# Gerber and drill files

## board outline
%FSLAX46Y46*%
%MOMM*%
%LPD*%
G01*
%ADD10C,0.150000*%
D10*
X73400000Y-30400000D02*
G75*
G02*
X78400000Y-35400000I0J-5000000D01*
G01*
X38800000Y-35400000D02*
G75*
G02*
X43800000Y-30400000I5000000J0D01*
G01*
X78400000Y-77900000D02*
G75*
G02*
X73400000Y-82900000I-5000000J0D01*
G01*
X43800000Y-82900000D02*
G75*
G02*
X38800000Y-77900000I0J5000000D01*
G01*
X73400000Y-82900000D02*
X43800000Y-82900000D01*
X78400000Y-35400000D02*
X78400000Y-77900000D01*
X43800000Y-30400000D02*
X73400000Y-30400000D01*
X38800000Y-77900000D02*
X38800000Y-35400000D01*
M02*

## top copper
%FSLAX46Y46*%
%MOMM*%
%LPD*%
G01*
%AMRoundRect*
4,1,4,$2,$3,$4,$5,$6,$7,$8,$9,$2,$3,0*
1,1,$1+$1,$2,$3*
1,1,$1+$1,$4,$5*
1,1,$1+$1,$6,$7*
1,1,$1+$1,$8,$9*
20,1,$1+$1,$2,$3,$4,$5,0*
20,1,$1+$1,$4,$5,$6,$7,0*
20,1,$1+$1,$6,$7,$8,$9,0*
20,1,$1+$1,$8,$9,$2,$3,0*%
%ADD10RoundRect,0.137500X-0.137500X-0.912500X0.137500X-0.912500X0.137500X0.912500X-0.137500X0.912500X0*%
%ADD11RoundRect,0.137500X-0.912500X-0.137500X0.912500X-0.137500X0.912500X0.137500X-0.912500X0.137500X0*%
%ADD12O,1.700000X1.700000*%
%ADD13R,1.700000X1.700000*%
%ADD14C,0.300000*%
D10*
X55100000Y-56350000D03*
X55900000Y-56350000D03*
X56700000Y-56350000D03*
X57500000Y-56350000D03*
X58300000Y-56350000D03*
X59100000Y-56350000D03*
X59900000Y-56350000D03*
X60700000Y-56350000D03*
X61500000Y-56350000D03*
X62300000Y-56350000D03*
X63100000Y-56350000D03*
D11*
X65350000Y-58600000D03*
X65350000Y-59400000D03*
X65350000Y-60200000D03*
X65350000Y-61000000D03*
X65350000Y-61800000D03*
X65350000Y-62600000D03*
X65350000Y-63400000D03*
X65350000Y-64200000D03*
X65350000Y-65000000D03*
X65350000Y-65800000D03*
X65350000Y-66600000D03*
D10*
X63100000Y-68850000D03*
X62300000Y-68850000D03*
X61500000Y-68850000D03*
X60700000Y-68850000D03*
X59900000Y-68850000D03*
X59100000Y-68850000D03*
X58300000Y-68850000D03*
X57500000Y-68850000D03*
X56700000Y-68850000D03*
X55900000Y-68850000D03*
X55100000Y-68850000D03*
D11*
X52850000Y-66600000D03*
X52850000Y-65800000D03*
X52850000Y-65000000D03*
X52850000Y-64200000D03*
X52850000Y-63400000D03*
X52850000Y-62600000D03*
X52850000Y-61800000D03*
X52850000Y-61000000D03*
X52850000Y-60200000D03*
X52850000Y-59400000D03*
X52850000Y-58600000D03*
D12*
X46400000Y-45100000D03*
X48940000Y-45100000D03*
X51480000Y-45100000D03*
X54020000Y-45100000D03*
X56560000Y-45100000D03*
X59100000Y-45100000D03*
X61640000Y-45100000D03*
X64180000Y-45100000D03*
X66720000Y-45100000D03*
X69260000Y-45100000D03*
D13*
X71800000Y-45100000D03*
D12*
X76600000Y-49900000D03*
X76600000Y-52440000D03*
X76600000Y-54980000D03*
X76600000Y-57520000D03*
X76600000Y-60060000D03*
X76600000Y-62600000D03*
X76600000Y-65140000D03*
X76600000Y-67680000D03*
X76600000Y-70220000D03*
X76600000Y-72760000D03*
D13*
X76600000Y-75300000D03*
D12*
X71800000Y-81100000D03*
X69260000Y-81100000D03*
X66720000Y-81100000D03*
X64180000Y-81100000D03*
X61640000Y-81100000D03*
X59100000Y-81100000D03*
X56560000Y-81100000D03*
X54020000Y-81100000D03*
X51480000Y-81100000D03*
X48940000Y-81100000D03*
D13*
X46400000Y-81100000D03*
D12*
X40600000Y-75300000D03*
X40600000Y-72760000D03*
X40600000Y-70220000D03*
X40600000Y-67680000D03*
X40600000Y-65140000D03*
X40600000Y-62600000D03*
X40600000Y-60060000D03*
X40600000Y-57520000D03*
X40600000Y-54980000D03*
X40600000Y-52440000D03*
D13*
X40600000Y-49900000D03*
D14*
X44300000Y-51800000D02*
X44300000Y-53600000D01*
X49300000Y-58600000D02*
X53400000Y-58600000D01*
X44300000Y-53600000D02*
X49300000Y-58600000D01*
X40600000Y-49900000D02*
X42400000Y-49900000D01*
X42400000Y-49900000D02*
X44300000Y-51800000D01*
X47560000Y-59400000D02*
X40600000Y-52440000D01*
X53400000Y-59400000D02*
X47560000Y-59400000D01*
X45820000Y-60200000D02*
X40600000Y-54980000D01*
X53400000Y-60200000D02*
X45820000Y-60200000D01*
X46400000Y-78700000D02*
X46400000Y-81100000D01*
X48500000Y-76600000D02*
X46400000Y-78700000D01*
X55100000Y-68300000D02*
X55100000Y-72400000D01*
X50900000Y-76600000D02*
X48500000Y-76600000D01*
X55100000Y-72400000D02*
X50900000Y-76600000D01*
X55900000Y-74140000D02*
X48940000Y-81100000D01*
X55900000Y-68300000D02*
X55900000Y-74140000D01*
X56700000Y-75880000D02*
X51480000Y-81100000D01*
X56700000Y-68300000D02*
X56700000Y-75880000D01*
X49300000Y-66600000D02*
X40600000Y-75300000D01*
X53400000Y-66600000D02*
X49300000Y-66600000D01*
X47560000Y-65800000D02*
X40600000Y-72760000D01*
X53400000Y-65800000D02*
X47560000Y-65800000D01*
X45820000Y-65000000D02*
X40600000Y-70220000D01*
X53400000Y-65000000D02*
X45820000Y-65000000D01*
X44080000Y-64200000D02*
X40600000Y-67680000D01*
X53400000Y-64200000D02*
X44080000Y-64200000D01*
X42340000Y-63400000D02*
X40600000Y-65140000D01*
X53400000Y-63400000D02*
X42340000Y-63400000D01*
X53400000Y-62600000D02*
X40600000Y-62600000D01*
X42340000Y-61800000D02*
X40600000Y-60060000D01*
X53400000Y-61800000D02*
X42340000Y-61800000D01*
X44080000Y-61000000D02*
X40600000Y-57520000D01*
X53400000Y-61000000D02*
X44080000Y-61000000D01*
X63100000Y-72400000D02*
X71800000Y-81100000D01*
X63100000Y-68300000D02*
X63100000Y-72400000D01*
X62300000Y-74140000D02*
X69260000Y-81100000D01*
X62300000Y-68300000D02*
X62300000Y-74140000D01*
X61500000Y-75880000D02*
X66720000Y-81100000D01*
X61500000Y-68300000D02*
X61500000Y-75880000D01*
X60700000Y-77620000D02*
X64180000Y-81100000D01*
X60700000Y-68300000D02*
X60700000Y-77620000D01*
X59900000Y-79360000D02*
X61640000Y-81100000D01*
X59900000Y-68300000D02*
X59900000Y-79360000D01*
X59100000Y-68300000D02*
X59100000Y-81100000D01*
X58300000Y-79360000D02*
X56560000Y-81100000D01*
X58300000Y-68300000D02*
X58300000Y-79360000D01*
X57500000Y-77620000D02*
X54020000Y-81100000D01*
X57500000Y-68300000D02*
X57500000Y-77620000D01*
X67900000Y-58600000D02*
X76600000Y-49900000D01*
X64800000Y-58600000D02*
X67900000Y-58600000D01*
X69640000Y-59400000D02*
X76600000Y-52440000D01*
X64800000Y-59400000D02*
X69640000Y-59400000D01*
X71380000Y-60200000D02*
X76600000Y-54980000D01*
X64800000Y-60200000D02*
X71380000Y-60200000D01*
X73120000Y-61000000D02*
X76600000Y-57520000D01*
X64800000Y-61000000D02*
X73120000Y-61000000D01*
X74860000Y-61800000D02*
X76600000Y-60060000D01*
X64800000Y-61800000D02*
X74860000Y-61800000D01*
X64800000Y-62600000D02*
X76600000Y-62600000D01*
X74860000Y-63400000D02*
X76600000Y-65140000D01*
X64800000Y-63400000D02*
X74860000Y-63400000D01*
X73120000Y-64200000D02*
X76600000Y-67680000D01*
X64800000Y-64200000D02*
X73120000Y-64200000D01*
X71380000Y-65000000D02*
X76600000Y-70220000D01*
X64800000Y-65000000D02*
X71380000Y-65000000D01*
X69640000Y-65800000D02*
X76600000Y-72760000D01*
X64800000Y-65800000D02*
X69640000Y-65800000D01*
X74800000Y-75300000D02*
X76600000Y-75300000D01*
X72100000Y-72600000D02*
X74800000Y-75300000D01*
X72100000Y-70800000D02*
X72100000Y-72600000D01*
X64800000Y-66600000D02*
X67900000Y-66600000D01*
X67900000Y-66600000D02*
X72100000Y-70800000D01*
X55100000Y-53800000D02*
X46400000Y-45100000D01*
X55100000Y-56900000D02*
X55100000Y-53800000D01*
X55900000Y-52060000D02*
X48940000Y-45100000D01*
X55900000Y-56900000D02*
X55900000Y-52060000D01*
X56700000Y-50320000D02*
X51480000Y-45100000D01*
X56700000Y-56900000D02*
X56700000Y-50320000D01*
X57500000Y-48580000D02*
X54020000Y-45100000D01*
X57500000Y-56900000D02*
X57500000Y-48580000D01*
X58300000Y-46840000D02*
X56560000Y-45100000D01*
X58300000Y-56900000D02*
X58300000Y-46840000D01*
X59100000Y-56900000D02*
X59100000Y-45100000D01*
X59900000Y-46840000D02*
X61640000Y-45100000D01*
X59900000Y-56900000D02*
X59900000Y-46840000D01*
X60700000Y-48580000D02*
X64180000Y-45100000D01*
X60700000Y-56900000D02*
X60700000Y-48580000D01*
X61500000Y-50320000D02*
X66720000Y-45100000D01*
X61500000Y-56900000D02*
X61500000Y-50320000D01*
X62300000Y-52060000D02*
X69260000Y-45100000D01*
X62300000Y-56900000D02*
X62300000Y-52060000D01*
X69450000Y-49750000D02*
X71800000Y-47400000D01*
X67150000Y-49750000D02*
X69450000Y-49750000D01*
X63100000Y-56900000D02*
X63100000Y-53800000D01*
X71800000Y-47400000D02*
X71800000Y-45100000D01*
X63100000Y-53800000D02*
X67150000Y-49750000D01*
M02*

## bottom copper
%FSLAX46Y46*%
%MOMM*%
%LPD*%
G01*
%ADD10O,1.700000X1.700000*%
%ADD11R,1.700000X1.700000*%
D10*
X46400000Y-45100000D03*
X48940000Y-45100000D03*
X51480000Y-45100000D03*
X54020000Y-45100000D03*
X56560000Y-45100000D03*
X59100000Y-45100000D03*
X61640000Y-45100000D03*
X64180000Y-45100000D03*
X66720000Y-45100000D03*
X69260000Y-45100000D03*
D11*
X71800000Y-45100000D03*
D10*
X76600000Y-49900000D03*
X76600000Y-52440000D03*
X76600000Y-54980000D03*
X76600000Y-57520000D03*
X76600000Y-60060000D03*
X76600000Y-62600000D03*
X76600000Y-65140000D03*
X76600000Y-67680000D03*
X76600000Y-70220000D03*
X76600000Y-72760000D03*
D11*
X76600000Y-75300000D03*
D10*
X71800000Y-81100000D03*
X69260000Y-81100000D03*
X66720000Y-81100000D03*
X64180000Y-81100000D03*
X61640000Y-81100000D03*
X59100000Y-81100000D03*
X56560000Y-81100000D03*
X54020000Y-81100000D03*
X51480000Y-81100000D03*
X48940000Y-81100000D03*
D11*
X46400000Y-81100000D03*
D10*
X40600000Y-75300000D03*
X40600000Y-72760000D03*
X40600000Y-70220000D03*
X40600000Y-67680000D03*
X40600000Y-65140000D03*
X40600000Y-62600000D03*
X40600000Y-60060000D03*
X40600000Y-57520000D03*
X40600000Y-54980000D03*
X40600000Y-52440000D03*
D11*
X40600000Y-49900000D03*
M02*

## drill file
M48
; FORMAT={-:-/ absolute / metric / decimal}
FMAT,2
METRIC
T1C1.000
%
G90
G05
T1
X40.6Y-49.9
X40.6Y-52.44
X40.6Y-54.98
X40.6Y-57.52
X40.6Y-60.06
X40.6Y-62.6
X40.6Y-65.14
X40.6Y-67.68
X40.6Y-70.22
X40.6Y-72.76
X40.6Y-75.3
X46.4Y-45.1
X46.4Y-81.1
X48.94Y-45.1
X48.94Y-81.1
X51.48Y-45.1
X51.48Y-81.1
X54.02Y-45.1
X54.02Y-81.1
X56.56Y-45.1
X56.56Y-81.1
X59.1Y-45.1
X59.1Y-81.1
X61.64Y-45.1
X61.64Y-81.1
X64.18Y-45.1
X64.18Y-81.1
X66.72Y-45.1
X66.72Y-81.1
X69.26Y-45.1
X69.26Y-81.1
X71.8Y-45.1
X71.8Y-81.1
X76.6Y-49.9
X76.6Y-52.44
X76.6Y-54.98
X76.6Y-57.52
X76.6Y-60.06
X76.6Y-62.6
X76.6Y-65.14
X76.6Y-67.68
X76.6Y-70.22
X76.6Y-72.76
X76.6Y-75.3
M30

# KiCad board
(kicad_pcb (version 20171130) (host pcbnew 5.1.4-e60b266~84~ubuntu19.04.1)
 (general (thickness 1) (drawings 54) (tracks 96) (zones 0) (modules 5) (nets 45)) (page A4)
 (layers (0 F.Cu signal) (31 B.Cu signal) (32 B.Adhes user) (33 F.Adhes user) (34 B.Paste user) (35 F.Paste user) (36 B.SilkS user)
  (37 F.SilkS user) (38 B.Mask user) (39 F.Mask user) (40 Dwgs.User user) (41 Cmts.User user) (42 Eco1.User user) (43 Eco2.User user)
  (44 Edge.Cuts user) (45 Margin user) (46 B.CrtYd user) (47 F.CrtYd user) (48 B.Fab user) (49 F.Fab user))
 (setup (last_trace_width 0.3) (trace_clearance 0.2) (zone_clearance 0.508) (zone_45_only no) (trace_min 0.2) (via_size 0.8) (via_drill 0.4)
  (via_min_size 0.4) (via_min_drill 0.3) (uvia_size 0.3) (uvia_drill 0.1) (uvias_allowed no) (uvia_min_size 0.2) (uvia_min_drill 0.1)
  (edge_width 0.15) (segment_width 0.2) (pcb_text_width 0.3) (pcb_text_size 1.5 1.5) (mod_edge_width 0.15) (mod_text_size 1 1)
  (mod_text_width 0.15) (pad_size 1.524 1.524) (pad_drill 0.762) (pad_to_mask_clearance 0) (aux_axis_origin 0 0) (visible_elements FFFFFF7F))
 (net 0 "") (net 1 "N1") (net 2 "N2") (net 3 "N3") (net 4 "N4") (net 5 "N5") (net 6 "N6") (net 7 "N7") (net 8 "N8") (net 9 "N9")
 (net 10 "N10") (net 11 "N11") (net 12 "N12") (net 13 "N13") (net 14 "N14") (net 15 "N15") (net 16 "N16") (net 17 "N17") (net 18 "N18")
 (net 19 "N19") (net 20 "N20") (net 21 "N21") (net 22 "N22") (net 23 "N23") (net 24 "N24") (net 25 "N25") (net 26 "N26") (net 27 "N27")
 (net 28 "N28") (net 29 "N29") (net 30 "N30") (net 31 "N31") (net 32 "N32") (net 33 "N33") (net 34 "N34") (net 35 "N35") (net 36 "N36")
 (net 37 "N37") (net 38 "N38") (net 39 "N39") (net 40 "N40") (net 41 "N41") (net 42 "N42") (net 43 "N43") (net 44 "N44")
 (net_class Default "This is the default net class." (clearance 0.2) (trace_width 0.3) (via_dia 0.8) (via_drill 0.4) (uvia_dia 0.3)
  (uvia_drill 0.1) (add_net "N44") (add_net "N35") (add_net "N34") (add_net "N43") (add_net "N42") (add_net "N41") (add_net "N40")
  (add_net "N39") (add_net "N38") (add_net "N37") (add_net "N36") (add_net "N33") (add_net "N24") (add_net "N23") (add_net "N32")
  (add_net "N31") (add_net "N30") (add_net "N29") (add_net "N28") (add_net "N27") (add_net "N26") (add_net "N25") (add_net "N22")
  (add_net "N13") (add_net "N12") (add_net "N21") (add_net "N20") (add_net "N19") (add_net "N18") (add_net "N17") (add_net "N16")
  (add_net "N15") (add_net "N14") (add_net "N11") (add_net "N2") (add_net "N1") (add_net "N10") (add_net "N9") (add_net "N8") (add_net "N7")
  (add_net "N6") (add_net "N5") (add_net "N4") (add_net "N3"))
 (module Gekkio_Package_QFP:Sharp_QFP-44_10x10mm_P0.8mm (layer F.Cu) (at 59.1 62.6)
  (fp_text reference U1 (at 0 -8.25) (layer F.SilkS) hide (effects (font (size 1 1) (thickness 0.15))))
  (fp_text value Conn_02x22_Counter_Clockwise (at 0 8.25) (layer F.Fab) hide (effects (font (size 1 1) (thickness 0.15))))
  (pad 44 smd roundrect (at -4 -6.25) (size 0.55 2.1) (layers F.Cu F.Paste F.Mask) (roundrect_rratio 0.25) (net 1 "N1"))
  (pad 43 smd roundrect (at -3.2 -6.25) (size 0.55 2.1) (layers F.Cu F.Paste F.Mask) (roundrect_rratio 0.25) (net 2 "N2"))
  (pad 42 smd roundrect (at -2.4 -6.25) (size 0.55 2.1) (layers F.Cu F.Paste F.Mask) (roundrect_rratio 0.25) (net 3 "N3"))
  (pad 41 smd roundrect (at -1.6 -6.25) (size 0.55 2.1) (layers F.Cu F.Paste F.Mask) (roundrect_rratio 0.25) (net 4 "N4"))
  (pad 40 smd roundrect (at -0.8 -6.25) (size 0.55 2.1) (layers F.Cu F.Paste F.Mask) (roundrect_rratio 0.25) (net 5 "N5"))
  (pad 39 smd roundrect (at 0 -6.25) (size 0.55 2.1) (layers F.Cu F.Paste F.Mask) (roundrect_rratio 0.25) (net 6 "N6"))
  (pad 38 smd roundrect (at 0.8 -6.25) (size 0.55 2.1) (layers F.Cu F.Paste F.Mask) (roundrect_rratio 0.25) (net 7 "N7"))
  (pad 37 smd roundrect (at 1.6 -6.25) (size 0.55 2.1) (layers F.Cu F.Paste F.Mask) (roundrect_rratio 0.25) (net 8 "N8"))
  (pad 36 smd roundrect (at 2.4 -6.25) (size 0.55 2.1) (layers F.Cu F.Paste F.Mask) (roundrect_rratio 0.25) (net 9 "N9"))
  (pad 35 smd roundrect (at 3.2 -6.25) (size 0.55 2.1) (layers F.Cu F.Paste F.Mask) (roundrect_rratio 0.25) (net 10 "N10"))
  (pad 34 smd roundrect (at 4 -6.25) (size 0.55 2.1) (layers F.Cu F.Paste F.Mask) (roundrect_rratio 0.25) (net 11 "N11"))
  (pad 33 smd roundrect (at 6.25 -4) (size 2.1 0.55) (layers F.Cu F.Paste F.Mask) (roundrect_rratio 0.25) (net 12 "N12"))
  (pad 32 smd roundrect (at 6.25 -3.2) (size 2.1 0.55) (layers F.Cu F.Paste F.Mask) (roundrect_rratio 0.25) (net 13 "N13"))
  (pad 31 smd roundrect (at 6.25 -2.4) (size 2.1 0.55) (layers F.Cu F.Paste F.Mask) (roundrect_rratio 0.25) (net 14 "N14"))
  (pad 30 smd roundrect (at 6.25 -1.6) (size 2.1 0.55) (layers F.Cu F.Paste F.Mask) (roundrect_rratio 0.25) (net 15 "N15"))
  (pad 29 smd roundrect (at 6.25 -0.8) (size 2.1 0.55) (layers F.Cu F.Paste F.Mask) (roundrect_rratio 0.25) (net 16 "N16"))
  (pad 28 smd roundrect (at 6.25 0) (size 2.1 0.55) (layers F.Cu F.Paste F.Mask) (roundrect_rratio 0.25) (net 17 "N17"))
  (pad 27 smd roundrect (at 6.25 0.8) (size 2.1 0.55) (layers F.Cu F.Paste F.Mask) (roundrect_rratio 0.25) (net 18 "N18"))
  (pad 26 smd roundrect (at 6.25 1.6) (size 2.1 0.55) (layers F.Cu F.Paste F.Mask) (roundrect_rratio 0.25) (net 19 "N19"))
  (pad 25 smd roundrect (at 6.25 2.4) (size 2.1 0.55) (layers F.Cu F.Paste F.Mask) (roundrect_rratio 0.25) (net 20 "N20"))
  (pad 24 smd roundrect (at 6.25 3.2) (size 2.1 0.55) (layers F.Cu F.Paste F.Mask) (roundrect_rratio 0.25) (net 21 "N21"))
  (pad 23 smd roundrect (at 6.25 4) (size 2.1 0.55) (layers F.Cu F.Paste F.Mask) (roundrect_rratio 0.25) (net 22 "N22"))
  (pad 22 smd roundrect (at 4 6.25) (size 0.55 2.1) (layers F.Cu F.Paste F.Mask) (roundrect_rratio 0.25) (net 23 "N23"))
  (pad 21 smd roundrect (at 3.2 6.25) (size 0.55 2.1) (layers F.Cu F.Paste F.Mask) (roundrect_rratio 0.25) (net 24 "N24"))
  (pad 20 smd roundrect (at 2.4 6.25) (size 0.55 2.1) (layers F.Cu F.Paste F.Mask) (roundrect_rratio 0.25) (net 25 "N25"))
  (pad 19 smd roundrect (at 1.6 6.25) (size 0.55 2.1) (layers F.Cu F.Paste F.Mask) (roundrect_rratio 0.25) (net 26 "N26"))
  (pad 18 smd roundrect (at 0.8 6.25) (size 0.55 2.1) (layers F.Cu F.Paste F.Mask) (roundrect_rratio 0.25) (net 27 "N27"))
  (pad 17 smd roundrect (at 0 6.25) (size 0.55 2.1) (layers F.Cu F.Paste F.Mask) (roundrect_rratio 0.25) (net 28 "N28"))
  (pad 16 smd roundrect (at -0.8 6.25) (size 0.55 2.1) (layers F.Cu F.Paste F.Mask) (roundrect_rratio 0.25) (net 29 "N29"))
  (pad 15 smd roundrect (at -1.6 6.25) (size 0.55 2.1) (layers F.Cu F.Paste F.Mask) (roundrect_rratio 0.25) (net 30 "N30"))
  (pad 14 smd roundrect (at -2.4 6.25) (size 0.55 2.1) (layers F.Cu F.Paste F.Mask) (roundrect_rratio 0.25) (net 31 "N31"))
  (pad 13 smd roundrect (at -3.2 6.25) (size 0.55 2.1) (layers F.Cu F.Paste F.Mask) (roundrect_rratio 0.25) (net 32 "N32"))
  (pad 12 smd roundrect (at -4 6.25) (size 0.55 2.1) (layers F.Cu F.Paste F.Mask) (roundrect_rratio 0.25) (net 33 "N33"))
  (pad 11 smd roundrect (at -6.25 4) (size 2.1 0.55) (layers F.Cu F.Paste F.Mask) (roundrect_rratio 0.25) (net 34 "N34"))
  (pad 10 smd roundrect (at -6.25 3.2) (size 2.1 0.55) (layers F.Cu F.Paste F.Mask) (roundrect_rratio 0.25) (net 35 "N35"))
  (pad 9 smd roundrect (at -6.25 2.4) (size 2.1 0.55) (layers F.Cu F.Paste F.Mask) (roundrect_rratio 0.25) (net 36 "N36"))
  (pad 8 smd roundrect (at -6.25 1.6) (size 2.1 0.55) (layers F.Cu F.Paste F.Mask) (roundrect_rratio 0.25) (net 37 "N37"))
  (pad 7 smd roundrect (at -6.25 0.8) (size 2.1 0.55) (layers F.Cu F.Paste F.Mask) (roundrect_rratio 0.25) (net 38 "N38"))
  (pad 6 smd roundrect (at -6.25 0) (size 2.1 0.55) (layers F.Cu F.Paste F.Mask) (roundrect_rratio 0.25) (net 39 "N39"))
  (pad 5 smd roundrect (at -6.25 -0.8) (size 2.1 0.55) (layers F.Cu F.Paste F.Mask) (roundrect_rratio 0.25) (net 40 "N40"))
  (pad 4 smd roundrect (at -6.25 -1.6) (size 2.1 0.55) (layers F.Cu F.Paste F.Mask) (roundrect_rratio 0.25) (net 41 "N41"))
  (pad 3 smd roundrect (at -6.25 -2.4) (size 2.1 0.55) (layers F.Cu F.Paste F.Mask) (roundrect_rratio 0.25) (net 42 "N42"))
  (pad 2 smd roundrect (at -6.25 -3.2) (size 2.1 0.55) (layers F.Cu F.Paste F.Mask) (roundrect_rratio 0.25) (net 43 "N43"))
  (pad 1 smd roundrect (at -6.25 -4) (size 2.1 0.55) (layers F.Cu F.Paste F.Mask) (roundrect_rratio 0.25) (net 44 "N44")))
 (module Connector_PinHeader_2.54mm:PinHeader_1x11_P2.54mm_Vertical (layer F.Cu) (at 71.8 45.1 270)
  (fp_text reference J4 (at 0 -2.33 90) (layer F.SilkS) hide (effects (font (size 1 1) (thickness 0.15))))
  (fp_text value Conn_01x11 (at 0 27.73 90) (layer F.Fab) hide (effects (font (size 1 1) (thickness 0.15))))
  (pad 11 thru_hole oval (at 0 25.4 270) (size 1.7 1.7) (drill 1) (layers *.Cu *.Mask) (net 1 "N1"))
  (pad 10 thru_hole oval (at 0 22.86 270) (size 1.7 1.7) (drill 1) (layers *.Cu *.Mask) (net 2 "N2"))
  (pad 9 thru_hole oval (at 0 20.32 270) (size 1.7 1.7) (drill 1) (layers *.Cu *.Mask) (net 3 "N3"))
  (pad 8 thru_hole oval (at 0 17.78 270) (size 1.7 1.7) (drill 1) (layers *.Cu *.Mask) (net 4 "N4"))
  (pad 7 thru_hole oval (at 0 15.24 270) (size 1.7 1.7) (drill 1) (layers *.Cu *.Mask) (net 5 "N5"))
  (pad 6 thru_hole oval (at 0 12.7 270) (size 1.7 1.7) (drill 1) (layers *.Cu *.Mask) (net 6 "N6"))
  (pad 5 thru_hole oval (at 0 10.16 270) (size 1.7 1.7) (drill 1) (layers *.Cu *.Mask) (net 7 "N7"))
  (pad 4 thru_hole oval (at 0 7.62 270) (size 1.7 1.7) (drill 1) (layers *.Cu *.Mask) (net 8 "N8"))
  (pad 3 thru_hole oval (at 0 5.08 270) (size 1.7 1.7) (drill 1) (layers *.Cu *.Mask) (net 9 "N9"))
  (pad 2 thru_hole oval (at 0 2.54 270) (size 1.7 1.7) (drill 1) (layers *.Cu *.Mask) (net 10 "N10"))
  (pad 1 thru_hole rect (at 0 0 270) (size 1.7 1.7) (drill 1) (layers *.Cu *.Mask) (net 11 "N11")))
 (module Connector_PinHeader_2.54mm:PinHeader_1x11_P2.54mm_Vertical (layer F.Cu) (at 76.6 75.3 180)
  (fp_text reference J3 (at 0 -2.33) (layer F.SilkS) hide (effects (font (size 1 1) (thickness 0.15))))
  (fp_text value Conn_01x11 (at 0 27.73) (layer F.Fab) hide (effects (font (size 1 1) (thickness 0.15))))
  (pad 11 thru_hole oval (at 0 25.4 180) (size 1.7 1.7) (drill 1) (layers *.Cu *.Mask) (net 12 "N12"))
  (pad 10 thru_hole oval (at 0 22.86 180) (size 1.7 1.7) (drill 1) (layers *.Cu *.Mask) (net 13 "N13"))
  (pad 9 thru_hole oval (at 0 20.32 180) (size 1.7 1.7) (drill 1) (layers *.Cu *.Mask) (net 14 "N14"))
  (pad 8 thru_hole oval (at 0 17.78 180) (size 1.7 1.7) (drill 1) (layers *.Cu *.Mask) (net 15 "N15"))
  (pad 7 thru_hole oval (at 0 15.24 180) (size 1.7 1.7) (drill 1) (layers *.Cu *.Mask) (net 16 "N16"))
  (pad 6 thru_hole oval (at 0 12.7 180) (size 1.7 1.7) (drill 1) (layers *.Cu *.Mask) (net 17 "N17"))
  (pad 5 thru_hole oval (at 0 10.16 180) (size 1.7 1.7) (drill 1) (layers *.Cu *.Mask) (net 18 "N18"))
  (pad 4 thru_hole oval (at 0 7.62 180) (size 1.7 1.7) (drill 1) (layers *.Cu *.Mask) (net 19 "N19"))
  (pad 3 thru_hole oval (at 0 5.08 180) (size 1.7 1.7) (drill 1) (layers *.Cu *.Mask) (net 20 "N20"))
  (pad 2 thru_hole oval (at 0 2.54 180) (size 1.7 1.7) (drill 1) (layers *.Cu *.Mask) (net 21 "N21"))
  (pad 1 thru_hole rect (at 0 0 180) (size 1.7 1.7) (drill 1) (layers *.Cu *.Mask) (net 22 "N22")))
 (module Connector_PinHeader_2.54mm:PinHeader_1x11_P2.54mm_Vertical (layer F.Cu) (at 46.4 81.1 90)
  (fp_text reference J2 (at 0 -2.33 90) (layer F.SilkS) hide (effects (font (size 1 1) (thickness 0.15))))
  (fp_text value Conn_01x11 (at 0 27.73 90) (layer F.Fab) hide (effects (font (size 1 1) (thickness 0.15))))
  (pad 11 thru_hole oval (at 0 25.4 90) (size 1.7 1.7) (drill 1) (layers *.Cu *.Mask) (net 23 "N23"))
  (pad 10 thru_hole oval (at 0 22.86 90) (size 1.7 1.7) (drill 1) (layers *.Cu *.Mask) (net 24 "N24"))
  (pad 9 thru_hole oval (at 0 20.32 90) (size 1.7 1.7) (drill 1) (layers *.Cu *.Mask) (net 25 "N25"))
  (pad 8 thru_hole oval (at 0 17.78 90) (size 1.7 1.7) (drill 1) (layers *.Cu *.Mask) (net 26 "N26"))
  (pad 7 thru_hole oval (at 0 15.24 90) (size 1.7 1.7) (drill 1) (layers *.Cu *.Mask) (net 27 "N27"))
  (pad 6 thru_hole oval (at 0 12.7 90) (size 1.7 1.7) (drill 1) (layers *.Cu *.Mask) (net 28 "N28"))
  (pad 5 thru_hole oval (at 0 10.16 90) (size 1.7 1.7) (drill 1) (layers *.Cu *.Mask) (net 29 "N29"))
  (pad 4 thru_hole oval (at 0 7.62 90) (size 1.7 1.7) (drill 1) (layers *.Cu *.Mask) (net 30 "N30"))
  (pad 3 thru_hole oval (at 0 5.08 90) (size 1.7 1.7) (drill 1) (layers *.Cu *.Mask) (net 31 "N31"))
  (pad 2 thru_hole oval (at 0 2.54 90) (size 1.7 1.7) (drill 1) (layers *.Cu *.Mask) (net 32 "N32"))
  (pad 1 thru_hole rect (at 0 0 90) (size 1.7 1.7) (drill 1) (layers *.Cu *.Mask) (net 33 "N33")))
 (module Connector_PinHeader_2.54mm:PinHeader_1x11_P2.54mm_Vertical (layer F.Cu) (at 40.6 49.9)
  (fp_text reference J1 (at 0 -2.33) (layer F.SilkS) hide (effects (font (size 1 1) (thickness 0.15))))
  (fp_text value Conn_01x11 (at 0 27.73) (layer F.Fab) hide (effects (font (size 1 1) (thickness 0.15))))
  (pad 11 thru_hole oval (at 0 25.4) (size 1.7 1.7) (drill 1) (layers *.Cu *.Mask) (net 34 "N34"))
  (pad 10 thru_hole oval (at 0 22.86) (size 1.7 1.7) (drill 1) (layers *.Cu *.Mask) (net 35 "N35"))
  (pad 9 thru_hole oval (at 0 20.32) (size 1.7 1.7) (drill 1) (layers *.Cu *.Mask) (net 36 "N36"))
  (pad 8 thru_hole oval (at 0 17.78) (size 1.7 1.7) (drill 1) (layers *.Cu *.Mask) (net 37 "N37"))
  (pad 7 thru_hole oval (at 0 15.24) (size 1.7 1.7) (drill 1) (layers *.Cu *.Mask) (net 38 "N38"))
  (pad 6 thru_hole oval (at 0 12.7) (size 1.7 1.7) (drill 1) (layers *.Cu *.Mask) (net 39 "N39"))
  (pad 5 thru_hole oval (at 0 10.16) (size 1.7 1.7) (drill 1) (layers *.Cu *.Mask) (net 40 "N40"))
  (pad 4 thru_hole oval (at 0 7.62) (size 1.7 1.7) (drill 1) (layers *.Cu *.Mask) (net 41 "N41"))
  (pad 3 thru_hole oval (at 0 5.08) (size 1.7 1.7) (drill 1) (layers *.Cu *.Mask) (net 42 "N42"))
  (pad 2 thru_hole oval (at 0 2.54) (size 1.7 1.7) (drill 1) (layers *.Cu *.Mask) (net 43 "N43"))
  (pad 1 thru_hole rect (at 0 0) (size 1.7 1.7) (drill 1) (layers *.Cu *.Mask) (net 44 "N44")))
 (gr_arc (start 73.4 35.4) (end 78.4 35.4) (angle -90) (layer Edge.Cuts) (width 0.15))
 (gr_arc (start 43.8 35.4) (end 43.8 30.4) (angle -90) (layer Edge.Cuts) (width 0.15))
 (gr_arc (start 73.4 77.9) (end 73.4 82.9) (angle -90) (layer Edge.Cuts) (width 0.15))
 (gr_arc (start 43.8 77.9) (end 38.8 77.9) (angle -90) (layer Edge.Cuts) (width 0.15))
 (gr_line (start 73.4 82.9) (end 43.8 82.9) (layer Edge.Cuts) (width 0.15))
 (gr_line (start 78.4 35.4) (end 78.4 77.9) (layer Edge.Cuts) (width 0.15))
 (gr_line (start 43.8 30.4) (end 73.4 30.4) (layer Edge.Cuts) (width 0.15))
 (gr_line (start 38.8 77.9) (end 38.8 35.4) (layer Edge.Cuts) (width 0.15))
 (segment (start 44.3 51.8) (end 44.3 53.6) (width 0.3) (layer F.Cu) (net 44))
 (segment (start 49.3 58.6) (end 53.4 58.6) (width 0.3) (layer F.Cu) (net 44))
 (segment (start 44.3 53.6) (end 49.3 58.6) (width 0.3) (layer F.Cu) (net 44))
 (segment (start 40.6 49.9) (end 42.4 49.9) (width 0.3) (layer F.Cu) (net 44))
 (segment (start 42.4 49.9) (end 44.3 51.8) (width 0.3) (layer F.Cu) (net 44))
 (segment (start 47.56 59.4) (end 40.6 52.44) (width 0.3) (layer F.Cu) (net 43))
 (segment (start 53.4 59.4) (end 47.56 59.4) (width 0.3) (layer F.Cu) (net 43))
 (segment (start 45.82 60.2) (end 40.6 54.98) (width 0.3) (layer F.Cu) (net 42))
 (segment (start 53.4 60.2) (end 45.82 60.2) (width 0.3) (layer F.Cu) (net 42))
 (segment (start 46.4 78.7) (end 46.4 81.1) (width 0.3) (layer F.Cu) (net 33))
 (segment (start 48.5 76.6) (end 46.4 78.7) (width 0.3) (layer F.Cu) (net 33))
 (segment (start 55.1 68.3) (end 55.1 72.4) (width 0.3) (layer F.Cu) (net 33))
 (segment (start 50.9 76.6) (end 48.5 76.6) (width 0.3) (layer F.Cu) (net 33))
 (segment (start 55.1 72.4) (end 50.9 76.6) (width 0.3) (layer F.Cu) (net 33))
 (segment (start 55.9 74.14) (end 48.94 81.1) (width 0.3) (layer F.Cu) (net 32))
 (segment (start 55.9 68.3) (end 55.9 74.14) (width 0.3) (layer F.Cu) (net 32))
 (segment (start 56.7 75.88) (end 51.48 81.1) (width 0.3) (layer F.Cu) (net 31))
 (segment (start 56.7 68.3) (end 56.7 75.88) (width 0.3) (layer F.Cu) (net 31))
 (segment (start 49.3 66.6) (end 40.6 75.3) (width 0.3) (layer F.Cu) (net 34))
 (segment (start 53.4 66.6) (end 49.3 66.6) (width 0.3) (layer F.Cu) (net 34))
 (segment (start 47.56 65.8) (end 40.6 72.76) (width 0.3) (layer F.Cu) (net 35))
 (segment (start 53.4 65.8) (end 47.56 65.8) (width 0.3) (layer F.Cu) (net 35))
 (segment (start 45.82 65) (end 40.6 70.22) (width 0.3) (layer F.Cu) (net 36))
 (segment (start 53.4 65) (end 45.82 65) (width 0.3) (layer F.Cu) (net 36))
 (segment (start 44.08 64.2) (end 40.6 67.68) (width 0.3) (layer F.Cu) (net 37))
 (segment (start 53.4 64.2) (end 44.08 64.2) (width 0.3) (layer F.Cu) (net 37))
 (segment (start 42.34 63.4) (end 40.6 65.14) (width 0.3) (layer F.Cu) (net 38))
 (segment (start 53.4 63.4) (end 42.34 63.4) (width 0.3) (layer F.Cu) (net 38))
 (segment (start 53.4 62.6) (end 40.6 62.6) (width 0.3) (layer F.Cu) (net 39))
 (segment (start 42.34 61.8) (end 40.6 60.06) (width 0.3) (layer F.Cu) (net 40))
 (segment (start 53.4 61.8) (end 42.34 61.8) (width 0.3) (layer F.Cu) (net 40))
 (segment (start 44.08 61) (end 40.6 57.52) (width 0.3) (layer F.Cu) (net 41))
 (segment (start 53.4 61) (end 44.08 61) (width 0.3) (layer F.Cu) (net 41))
 (segment (start 63.1 72.4) (end 71.8 81.1) (width 0.3) (layer F.Cu) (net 23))
 (segment (start 63.1 68.3) (end 63.1 72.4) (width 0.3) (layer F.Cu) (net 23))
 (segment (start 62.3 74.14) (end 69.26 81.1) (width 0.3) (layer F.Cu) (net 24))
 (segment (start 62.3 68.3) (end 62.3 74.14) (width 0.3) (layer F.Cu) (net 24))
 (segment (start 61.5 75.88) (end 66.72 81.1) (width 0.3) (layer F.Cu) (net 25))
 (segment (start 61.5 68.3) (end 61.5 75.88) (width 0.3) (layer F.Cu) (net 25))
 (segment (start 60.7 77.62) (end 64.18 81.1) (width 0.3) (layer F.Cu) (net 26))
 (segment (start 60.7 68.3) (end 60.7 77.62) (width 0.3) (layer F.Cu) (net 26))
 (segment (start 59.9 79.36) (end 61.64 81.1) (width 0.3) (layer F.Cu) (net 27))
 (segment (start 59.9 68.3) (end 59.9 79.36) (width 0.3) (layer F.Cu) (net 27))
 (segment (start 59.1 68.3) (end 59.1 81.1) (width 0.3) (layer F.Cu) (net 28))
 (segment (start 58.3 79.36) (end 56.56 81.1) (width 0.3) (layer F.Cu) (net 29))
 (segment (start 58.3 68.3) (end 58.3 79.36) (width 0.3) (layer F.Cu) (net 29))
 (segment (start 57.5 77.62) (end 54.02 81.1) (width 0.3) (layer F.Cu) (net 30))
 (segment (start 57.5 68.3) (end 57.5 77.62) (width 0.3) (layer F.Cu) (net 30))
 (segment (start 67.9 58.6) (end 76.6 49.9) (width 0.3) (layer F.Cu) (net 12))
 (segment (start 64.8 58.6) (end 67.9 58.6) (width 0.3) (layer F.Cu) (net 12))
 (segment (start 69.64 59.4) (end 76.6 52.44) (width 0.3) (layer F.Cu) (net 13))
 (segment (start 64.8 59.4) (end 69.64 59.4) (width 0.3) (layer F.Cu) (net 13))
 (segment (start 71.38 60.2) (end 76.6 54.98) (width 0.3) (layer F.Cu) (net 14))
 (segment (start 64.8 60.2) (end 71.38 60.2) (width 0.3) (layer F.Cu) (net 14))
 (segment (start 73.12 61) (end 76.6 57.52) (width 0.3) (layer F.Cu) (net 15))
 (segment (start 64.8 61) (end 73.12 61) (width 0.3) (layer F.Cu) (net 15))
 (segment (start 74.86 61.8) (end 76.6 60.06) (width 0.3) (layer F.Cu) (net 16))
 (segment (start 64.8 61.8) (end 74.86 61.8) (width 0.3) (layer F.Cu) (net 16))
 (segment (start 64.8 62.6) (end 76.6 62.6) (width 0.3) (layer F.Cu) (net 17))
 (segment (start 74.86 63.4) (end 76.6 65.14) (width 0.3) (layer F.Cu) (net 18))
 (segment (start 64.8 63.4) (end 74.86 63.4) (width 0.3) (layer F.Cu) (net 18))
 (segment (start 73.12 64.2) (end 76.6 67.68) (width 0.3) (layer F.Cu) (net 19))
 (segment (start 64.8 64.2) (end 73.12 64.2) (width 0.3) (layer F.Cu) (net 19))
 (segment (start 71.38 65) (end 76.6 70.22) (width 0.3) (layer F.Cu) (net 20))
 (segment (start 64.8 65) (end 71.38 65) (width 0.3) (layer F.Cu) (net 20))
 (segment (start 69.64 65.8) (end 76.6 72.76) (width 0.3) (layer F.Cu) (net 21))
 (segment (start 64.8 65.8) (end 69.64 65.8) (width 0.3) (layer F.Cu) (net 21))
 (segment (start 74.8 75.3) (end 76.6 75.3) (width 0.3) (layer F.Cu) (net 22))
 (segment (start 72.1 72.6) (end 74.8 75.3) (width 0.3) (layer F.Cu) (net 22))
 (segment (start 72.1 70.8) (end 72.1 72.6) (width 0.3) (layer F.Cu) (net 22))
 (segment (start 64.8 66.6) (end 67.9 66.6) (width 0.3) (layer F.Cu) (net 22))
 (segment (start 67.9 66.6) (end 72.1 70.8) (width 0.3) (layer F.Cu) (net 22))
 (segment (start 55.1 53.8) (end 46.4 45.1) (width 0.3) (layer F.Cu) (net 1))
 (segment (start 55.1 56.9) (end 55.1 53.8) (width 0.3) (layer F.Cu) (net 1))
 (segment (start 55.9 52.06) (end 48.94 45.1) (width 0.3) (layer F.Cu) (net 2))
 (segment (start 55.9 56.9) (end 55.9 52.06) (width 0.3) (layer F.Cu) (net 2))
 (segment (start 56.7 50.32) (end 51.48 45.1) (width 0.3) (layer F.Cu) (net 3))
 (segment (start 56.7 56.9) (end 56.7 50.32) (width 0.3) (layer F.Cu) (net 3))
 (segment (start 57.5 48.58) (end 54.02 45.1) (width 0.3) (layer F.Cu) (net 4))
 (segment (start 57.5 56.9) (end 57.5 48.58) (width 0.3) (layer F.Cu) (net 4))
 (segment (start 58.3 46.84) (end 56.56 45.1) (width 0.3) (layer F.Cu) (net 5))
 (segment (start 58.3 56.9) (end 58.3 46.84) (width 0.3) (layer F.Cu) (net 5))
 (segment (start 59.1 56.9) (end 59.1 45.1) (width 0.3) (layer F.Cu) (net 6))
 (segment (start 59.9 46.84) (end 61.64 45.1) (width 0.3) (layer F.Cu) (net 7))
 (segment (start 59.9 56.9) (end 59.9 46.84) (width 0.3) (layer F.Cu) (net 7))
 (segment (start 60.7 48.58) (end 64.18 45.1) (width 0.3) (layer F.Cu) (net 8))
 (segment (start 60.7 56.9) (end 60.7 48.58) (width 0.3) (layer F.Cu) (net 8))
 (segment (start 61.5 50.32) (end 66.72 45.1) (width 0.3) (layer F.Cu) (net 9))
 (segment (start 61.5 56.9) (end 61.5 50.32) (width 0.3) (layer F.Cu) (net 9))
 (segment (start 62.3 52.06) (end 69.26 45.1) (width 0.3) (layer F.Cu) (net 10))
 (segment (start 62.3 56.9) (end 62.3 52.06) (width 0.3) (layer F.Cu) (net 10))
 (segment (start 69.45 49.75) (end 71.8 47.4) (width 0.3) (layer F.Cu) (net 11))
 (segment (start 67.15 49.75) (end 69.45 49.75) (width 0.3) (layer F.Cu) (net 11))
 (segment (start 63.1 56.9) (end 63.1 53.8) (width 0.3) (layer F.Cu) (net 11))
 (segment (start 71.8 47.4) (end 71.8 45.1) (width 0.3) (layer F.Cu) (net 11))
 (segment (start 63.1 53.8) (end 67.15 49.75) (width 0.3) (layer F.Cu) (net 11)))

